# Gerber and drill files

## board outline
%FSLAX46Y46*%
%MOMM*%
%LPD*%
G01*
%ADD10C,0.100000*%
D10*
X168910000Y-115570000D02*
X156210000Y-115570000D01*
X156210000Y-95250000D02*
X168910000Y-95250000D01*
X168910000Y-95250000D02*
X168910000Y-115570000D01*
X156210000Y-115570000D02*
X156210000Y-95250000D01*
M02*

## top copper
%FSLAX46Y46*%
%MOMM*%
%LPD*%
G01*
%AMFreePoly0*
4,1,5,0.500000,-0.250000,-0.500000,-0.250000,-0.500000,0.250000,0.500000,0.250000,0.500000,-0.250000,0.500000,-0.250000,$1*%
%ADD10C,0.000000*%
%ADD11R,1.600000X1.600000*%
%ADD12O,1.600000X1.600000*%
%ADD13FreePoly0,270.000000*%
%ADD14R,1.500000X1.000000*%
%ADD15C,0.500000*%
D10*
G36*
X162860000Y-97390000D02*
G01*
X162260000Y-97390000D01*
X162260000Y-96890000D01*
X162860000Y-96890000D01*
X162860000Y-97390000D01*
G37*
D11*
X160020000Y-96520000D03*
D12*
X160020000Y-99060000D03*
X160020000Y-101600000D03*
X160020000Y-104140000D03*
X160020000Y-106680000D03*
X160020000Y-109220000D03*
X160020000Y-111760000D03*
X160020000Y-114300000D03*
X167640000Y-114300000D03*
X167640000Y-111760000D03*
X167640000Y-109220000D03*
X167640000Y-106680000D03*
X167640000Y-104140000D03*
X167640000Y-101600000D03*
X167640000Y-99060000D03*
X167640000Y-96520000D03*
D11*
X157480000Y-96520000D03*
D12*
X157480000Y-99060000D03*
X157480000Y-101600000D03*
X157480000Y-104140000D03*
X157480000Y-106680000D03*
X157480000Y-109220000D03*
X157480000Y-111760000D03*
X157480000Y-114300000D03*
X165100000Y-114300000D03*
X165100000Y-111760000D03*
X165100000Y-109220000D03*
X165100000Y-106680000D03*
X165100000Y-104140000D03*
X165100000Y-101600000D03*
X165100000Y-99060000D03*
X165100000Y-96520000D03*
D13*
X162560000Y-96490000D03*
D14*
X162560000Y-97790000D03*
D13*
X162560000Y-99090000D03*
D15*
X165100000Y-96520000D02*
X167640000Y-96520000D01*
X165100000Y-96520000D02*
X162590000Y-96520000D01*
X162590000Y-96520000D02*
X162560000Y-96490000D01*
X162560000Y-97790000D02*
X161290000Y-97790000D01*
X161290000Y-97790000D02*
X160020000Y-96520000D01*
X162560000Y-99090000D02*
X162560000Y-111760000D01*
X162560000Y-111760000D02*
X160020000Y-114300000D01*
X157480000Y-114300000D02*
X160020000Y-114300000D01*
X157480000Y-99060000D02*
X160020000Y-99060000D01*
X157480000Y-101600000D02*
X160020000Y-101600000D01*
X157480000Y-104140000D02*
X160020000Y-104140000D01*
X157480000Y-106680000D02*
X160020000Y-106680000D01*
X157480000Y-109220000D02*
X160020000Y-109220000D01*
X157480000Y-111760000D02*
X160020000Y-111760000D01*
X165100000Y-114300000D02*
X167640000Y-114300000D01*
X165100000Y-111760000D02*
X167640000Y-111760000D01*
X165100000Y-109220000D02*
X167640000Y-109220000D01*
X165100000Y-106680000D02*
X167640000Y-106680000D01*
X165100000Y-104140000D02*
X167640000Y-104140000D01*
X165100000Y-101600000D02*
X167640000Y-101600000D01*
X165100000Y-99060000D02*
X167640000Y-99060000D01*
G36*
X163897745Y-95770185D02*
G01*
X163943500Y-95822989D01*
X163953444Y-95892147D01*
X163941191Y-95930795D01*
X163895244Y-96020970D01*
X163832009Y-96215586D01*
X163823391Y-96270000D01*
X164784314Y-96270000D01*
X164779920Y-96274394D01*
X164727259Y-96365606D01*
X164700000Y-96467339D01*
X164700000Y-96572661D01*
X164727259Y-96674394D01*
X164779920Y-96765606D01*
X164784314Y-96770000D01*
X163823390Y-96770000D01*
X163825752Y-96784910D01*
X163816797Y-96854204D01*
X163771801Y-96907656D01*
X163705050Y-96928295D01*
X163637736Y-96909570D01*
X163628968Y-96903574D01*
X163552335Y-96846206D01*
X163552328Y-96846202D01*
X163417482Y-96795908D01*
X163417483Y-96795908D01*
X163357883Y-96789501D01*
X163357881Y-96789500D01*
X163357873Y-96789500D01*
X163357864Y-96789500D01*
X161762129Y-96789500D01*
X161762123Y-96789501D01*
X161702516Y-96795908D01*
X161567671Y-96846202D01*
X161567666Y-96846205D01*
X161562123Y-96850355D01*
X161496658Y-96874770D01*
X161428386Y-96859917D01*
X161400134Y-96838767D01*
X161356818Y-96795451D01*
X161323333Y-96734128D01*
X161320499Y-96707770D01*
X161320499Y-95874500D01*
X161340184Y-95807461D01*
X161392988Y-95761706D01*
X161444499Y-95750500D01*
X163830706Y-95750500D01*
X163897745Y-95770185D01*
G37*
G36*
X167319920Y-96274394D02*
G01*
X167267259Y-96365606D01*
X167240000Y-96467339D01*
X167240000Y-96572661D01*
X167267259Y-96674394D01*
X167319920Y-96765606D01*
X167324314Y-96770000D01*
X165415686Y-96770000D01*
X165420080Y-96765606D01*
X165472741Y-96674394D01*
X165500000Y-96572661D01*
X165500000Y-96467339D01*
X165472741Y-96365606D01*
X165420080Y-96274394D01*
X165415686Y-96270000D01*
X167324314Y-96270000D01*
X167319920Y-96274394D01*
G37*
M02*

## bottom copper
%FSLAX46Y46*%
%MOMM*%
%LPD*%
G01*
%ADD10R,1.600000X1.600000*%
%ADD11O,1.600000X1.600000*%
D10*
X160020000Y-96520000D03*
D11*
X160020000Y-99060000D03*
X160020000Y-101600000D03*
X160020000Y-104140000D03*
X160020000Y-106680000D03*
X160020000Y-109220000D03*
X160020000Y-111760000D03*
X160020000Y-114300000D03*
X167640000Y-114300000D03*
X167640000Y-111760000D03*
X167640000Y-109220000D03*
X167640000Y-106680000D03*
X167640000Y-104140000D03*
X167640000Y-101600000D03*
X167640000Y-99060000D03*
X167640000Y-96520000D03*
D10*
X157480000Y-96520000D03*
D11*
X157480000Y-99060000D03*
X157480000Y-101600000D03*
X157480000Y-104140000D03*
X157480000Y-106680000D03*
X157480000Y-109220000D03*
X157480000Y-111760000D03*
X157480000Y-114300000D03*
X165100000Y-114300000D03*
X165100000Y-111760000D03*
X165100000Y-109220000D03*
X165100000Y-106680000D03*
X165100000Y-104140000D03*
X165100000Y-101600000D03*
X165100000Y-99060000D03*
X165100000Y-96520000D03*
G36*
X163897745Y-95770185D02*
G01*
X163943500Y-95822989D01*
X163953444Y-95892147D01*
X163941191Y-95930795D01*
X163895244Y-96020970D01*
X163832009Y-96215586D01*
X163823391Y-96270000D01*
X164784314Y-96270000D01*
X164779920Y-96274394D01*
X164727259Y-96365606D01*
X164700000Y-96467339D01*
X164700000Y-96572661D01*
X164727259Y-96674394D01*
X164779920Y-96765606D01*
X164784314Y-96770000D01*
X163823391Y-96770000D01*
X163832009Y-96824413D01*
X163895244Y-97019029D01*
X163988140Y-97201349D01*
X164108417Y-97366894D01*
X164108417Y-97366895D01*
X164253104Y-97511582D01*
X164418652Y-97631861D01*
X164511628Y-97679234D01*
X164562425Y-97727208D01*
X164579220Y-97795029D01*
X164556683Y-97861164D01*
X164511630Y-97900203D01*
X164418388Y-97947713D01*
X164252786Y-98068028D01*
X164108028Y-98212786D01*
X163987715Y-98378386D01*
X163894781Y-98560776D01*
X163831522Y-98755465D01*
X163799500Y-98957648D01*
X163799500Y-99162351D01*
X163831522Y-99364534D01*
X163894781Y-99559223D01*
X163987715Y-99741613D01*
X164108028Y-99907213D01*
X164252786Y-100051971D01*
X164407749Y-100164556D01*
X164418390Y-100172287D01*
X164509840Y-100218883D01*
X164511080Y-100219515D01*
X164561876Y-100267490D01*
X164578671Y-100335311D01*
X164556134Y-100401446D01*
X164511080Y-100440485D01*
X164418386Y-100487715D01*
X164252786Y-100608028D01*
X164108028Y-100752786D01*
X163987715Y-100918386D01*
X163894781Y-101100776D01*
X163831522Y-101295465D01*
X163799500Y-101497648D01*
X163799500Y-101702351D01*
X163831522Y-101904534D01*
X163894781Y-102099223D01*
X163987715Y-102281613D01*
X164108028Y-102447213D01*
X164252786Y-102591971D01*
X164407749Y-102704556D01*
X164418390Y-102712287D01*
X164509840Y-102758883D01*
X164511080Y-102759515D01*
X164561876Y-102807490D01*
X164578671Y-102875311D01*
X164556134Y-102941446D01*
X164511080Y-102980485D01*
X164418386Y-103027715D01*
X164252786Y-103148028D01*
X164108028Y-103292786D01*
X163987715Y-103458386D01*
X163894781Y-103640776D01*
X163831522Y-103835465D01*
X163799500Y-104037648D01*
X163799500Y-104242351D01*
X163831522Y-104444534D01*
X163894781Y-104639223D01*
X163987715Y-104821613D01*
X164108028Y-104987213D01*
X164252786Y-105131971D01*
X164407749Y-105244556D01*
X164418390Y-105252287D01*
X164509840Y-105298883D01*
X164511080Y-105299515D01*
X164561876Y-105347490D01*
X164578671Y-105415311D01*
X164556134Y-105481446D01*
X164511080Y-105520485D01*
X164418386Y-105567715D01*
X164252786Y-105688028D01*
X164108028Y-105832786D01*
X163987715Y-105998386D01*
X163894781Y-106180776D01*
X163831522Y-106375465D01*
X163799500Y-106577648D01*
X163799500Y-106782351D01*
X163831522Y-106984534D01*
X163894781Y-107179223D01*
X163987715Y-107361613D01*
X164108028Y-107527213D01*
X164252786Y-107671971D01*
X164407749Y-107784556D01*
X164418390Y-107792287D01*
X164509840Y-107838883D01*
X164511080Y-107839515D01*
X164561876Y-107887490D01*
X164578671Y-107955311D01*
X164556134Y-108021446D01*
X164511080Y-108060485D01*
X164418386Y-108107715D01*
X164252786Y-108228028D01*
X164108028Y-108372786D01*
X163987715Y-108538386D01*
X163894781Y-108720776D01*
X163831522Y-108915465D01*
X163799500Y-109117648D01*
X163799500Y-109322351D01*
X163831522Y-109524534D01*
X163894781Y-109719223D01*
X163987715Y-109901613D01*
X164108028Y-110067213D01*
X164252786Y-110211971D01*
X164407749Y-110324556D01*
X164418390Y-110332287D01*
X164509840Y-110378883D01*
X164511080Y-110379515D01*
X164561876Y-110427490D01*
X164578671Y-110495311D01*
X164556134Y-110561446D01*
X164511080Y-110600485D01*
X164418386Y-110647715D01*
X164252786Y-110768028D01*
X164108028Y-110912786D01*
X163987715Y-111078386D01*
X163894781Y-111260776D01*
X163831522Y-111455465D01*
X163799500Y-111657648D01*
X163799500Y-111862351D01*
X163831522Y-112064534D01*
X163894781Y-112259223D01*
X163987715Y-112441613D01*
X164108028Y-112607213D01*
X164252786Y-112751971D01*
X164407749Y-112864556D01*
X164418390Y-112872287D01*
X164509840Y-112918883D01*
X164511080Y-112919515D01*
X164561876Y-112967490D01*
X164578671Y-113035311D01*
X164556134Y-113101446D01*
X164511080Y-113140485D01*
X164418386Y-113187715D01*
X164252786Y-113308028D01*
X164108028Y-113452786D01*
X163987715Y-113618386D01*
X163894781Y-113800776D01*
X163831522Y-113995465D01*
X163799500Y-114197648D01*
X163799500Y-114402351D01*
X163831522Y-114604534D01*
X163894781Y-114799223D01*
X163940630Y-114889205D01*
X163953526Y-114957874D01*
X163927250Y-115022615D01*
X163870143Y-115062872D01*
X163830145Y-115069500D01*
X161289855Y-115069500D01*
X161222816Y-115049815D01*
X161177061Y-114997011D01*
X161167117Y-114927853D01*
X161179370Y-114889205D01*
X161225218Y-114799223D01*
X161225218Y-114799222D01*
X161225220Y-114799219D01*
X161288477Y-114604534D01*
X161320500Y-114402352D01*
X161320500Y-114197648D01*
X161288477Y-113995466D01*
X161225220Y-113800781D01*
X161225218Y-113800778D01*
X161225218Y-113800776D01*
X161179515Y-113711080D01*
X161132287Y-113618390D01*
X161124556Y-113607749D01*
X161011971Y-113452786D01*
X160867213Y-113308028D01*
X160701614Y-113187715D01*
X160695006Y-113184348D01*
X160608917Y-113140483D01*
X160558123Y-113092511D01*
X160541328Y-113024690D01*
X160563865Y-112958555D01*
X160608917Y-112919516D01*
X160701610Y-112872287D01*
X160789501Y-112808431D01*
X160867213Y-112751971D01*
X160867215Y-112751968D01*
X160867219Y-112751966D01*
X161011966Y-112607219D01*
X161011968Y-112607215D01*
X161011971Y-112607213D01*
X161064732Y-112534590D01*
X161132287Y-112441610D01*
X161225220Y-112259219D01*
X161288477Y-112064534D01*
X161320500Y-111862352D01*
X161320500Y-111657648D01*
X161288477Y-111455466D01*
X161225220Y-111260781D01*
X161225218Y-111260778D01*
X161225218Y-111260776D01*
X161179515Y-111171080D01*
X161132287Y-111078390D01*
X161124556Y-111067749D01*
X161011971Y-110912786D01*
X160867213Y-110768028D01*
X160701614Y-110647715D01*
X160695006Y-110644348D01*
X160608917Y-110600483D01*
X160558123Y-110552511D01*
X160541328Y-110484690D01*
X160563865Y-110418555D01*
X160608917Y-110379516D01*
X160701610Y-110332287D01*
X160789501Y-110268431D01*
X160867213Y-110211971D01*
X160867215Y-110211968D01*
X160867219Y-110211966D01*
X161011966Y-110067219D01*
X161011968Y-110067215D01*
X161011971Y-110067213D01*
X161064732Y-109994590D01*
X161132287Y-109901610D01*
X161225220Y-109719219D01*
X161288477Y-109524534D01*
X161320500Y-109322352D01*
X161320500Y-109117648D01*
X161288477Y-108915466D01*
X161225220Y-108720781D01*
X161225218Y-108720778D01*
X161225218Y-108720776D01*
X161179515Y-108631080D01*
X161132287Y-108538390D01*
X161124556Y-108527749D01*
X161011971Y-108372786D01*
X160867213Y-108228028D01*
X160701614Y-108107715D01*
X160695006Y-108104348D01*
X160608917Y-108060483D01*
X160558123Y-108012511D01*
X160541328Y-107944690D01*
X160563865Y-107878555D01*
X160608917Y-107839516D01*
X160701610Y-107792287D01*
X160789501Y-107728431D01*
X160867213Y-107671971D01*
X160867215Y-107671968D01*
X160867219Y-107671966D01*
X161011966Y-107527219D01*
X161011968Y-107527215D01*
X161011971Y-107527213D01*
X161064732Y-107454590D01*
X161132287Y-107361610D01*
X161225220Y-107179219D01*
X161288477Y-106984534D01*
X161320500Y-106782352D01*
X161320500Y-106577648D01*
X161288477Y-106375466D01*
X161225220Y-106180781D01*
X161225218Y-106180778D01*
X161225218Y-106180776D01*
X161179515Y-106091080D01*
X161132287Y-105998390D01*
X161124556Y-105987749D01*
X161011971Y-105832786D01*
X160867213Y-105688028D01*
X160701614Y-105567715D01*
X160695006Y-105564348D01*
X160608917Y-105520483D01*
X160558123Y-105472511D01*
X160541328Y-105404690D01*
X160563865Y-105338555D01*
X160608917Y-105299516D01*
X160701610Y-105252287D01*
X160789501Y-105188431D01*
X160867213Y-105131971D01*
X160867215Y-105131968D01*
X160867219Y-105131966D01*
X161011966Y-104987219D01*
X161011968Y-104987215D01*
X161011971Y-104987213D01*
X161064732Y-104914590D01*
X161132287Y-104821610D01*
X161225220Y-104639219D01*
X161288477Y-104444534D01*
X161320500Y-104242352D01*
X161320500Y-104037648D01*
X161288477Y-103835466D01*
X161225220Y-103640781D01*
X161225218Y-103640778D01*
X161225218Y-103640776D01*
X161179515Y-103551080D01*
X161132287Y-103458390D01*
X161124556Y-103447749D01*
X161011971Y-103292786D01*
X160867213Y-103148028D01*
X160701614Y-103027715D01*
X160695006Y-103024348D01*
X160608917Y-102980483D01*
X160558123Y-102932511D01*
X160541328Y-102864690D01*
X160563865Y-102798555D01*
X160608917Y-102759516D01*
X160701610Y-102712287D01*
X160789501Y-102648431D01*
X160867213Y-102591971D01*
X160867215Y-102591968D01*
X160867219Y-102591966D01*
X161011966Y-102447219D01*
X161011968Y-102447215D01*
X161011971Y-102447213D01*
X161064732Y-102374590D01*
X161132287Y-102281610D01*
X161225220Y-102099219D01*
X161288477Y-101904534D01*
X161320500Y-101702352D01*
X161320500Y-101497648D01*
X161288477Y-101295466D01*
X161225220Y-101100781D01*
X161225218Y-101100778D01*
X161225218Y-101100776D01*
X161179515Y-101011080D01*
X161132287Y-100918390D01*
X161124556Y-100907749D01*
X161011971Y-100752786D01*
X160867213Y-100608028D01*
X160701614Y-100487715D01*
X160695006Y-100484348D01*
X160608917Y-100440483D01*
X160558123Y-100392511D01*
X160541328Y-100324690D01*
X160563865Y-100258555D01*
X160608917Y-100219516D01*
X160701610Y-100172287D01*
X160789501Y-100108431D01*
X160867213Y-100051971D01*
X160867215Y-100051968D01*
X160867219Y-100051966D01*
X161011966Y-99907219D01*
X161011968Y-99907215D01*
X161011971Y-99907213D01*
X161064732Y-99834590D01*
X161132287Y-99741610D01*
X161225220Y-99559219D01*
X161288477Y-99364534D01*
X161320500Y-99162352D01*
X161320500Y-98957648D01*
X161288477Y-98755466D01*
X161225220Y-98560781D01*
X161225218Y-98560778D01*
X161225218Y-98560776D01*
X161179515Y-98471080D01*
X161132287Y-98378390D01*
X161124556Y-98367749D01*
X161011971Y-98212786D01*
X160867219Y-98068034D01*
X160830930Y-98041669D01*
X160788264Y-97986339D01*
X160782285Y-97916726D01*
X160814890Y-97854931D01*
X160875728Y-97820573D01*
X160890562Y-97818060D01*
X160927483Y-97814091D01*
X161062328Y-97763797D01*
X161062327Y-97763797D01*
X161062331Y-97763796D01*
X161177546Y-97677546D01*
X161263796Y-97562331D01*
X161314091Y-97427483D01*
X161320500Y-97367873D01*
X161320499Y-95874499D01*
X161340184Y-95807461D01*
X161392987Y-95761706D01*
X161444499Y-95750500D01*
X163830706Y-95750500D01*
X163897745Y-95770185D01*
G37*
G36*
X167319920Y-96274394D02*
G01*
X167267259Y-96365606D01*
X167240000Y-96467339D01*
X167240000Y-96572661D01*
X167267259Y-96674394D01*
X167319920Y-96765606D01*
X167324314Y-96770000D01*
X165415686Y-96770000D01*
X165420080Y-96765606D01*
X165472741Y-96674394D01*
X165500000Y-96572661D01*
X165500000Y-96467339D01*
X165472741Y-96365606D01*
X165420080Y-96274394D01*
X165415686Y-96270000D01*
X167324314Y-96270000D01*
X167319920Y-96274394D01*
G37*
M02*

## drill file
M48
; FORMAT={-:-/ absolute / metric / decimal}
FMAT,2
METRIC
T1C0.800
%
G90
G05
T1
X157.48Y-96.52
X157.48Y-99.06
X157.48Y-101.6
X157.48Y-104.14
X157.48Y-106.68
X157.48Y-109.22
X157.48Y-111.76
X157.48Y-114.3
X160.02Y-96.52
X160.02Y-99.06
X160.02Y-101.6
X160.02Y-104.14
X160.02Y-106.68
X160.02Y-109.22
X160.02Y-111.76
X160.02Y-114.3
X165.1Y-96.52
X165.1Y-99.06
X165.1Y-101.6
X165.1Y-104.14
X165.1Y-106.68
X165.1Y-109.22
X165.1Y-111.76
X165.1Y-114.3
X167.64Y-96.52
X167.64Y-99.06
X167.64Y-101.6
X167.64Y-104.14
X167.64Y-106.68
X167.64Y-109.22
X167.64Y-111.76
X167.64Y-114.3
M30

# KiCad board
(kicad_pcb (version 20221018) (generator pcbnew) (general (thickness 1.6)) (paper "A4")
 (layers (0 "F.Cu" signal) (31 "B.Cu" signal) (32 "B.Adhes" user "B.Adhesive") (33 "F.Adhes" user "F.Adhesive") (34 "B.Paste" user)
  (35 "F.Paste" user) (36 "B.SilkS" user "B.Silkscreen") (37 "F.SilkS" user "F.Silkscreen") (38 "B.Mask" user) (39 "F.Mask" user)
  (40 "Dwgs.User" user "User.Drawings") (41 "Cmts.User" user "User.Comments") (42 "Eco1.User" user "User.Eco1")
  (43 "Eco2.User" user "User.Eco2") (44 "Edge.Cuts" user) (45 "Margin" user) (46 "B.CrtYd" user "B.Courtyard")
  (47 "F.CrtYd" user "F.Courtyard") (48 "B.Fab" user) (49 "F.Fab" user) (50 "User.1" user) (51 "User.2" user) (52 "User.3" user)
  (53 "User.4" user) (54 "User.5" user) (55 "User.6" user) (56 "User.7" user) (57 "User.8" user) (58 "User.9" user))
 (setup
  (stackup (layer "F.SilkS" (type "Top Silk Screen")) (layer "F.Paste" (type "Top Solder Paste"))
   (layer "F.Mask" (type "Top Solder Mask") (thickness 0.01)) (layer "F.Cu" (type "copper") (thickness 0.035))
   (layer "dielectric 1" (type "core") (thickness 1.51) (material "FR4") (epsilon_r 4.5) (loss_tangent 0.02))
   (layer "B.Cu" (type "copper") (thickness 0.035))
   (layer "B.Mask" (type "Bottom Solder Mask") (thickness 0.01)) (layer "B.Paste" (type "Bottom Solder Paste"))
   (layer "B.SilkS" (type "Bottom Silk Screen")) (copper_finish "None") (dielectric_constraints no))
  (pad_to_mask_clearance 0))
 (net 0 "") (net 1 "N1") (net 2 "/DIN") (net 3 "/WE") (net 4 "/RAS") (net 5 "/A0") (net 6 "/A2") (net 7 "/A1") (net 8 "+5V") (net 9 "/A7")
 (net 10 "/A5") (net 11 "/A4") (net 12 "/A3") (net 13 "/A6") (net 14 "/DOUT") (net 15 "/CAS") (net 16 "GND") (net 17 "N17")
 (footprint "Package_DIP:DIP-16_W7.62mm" (layer "F.Cu") (at 160.02 96.52)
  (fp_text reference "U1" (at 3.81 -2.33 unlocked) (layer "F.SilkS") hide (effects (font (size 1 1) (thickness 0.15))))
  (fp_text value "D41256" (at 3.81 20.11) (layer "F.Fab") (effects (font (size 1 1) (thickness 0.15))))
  (pad "1" thru_hole rect (at 0 0) (size 1.6 1.6) (drill 0.8) (layers "*.Cu" "*.Mask") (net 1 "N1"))
  (pad "2" thru_hole oval (at 0 2.54) (size 1.6 1.6) (drill 0.8) (layers "*.Cu" "*.Mask") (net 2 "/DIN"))
  (pad "3" thru_hole oval (at 0 5.08) (size 1.6 1.6) (drill 0.8) (layers "*.Cu" "*.Mask") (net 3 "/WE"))
  (pad "4" thru_hole oval (at 0 7.62) (size 1.6 1.6) (drill 0.8) (layers "*.Cu" "*.Mask") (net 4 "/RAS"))
  (pad "5" thru_hole oval (at 0 10.16) (size 1.6 1.6) (drill 0.8) (layers "*.Cu" "*.Mask") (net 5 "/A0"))
  (pad "6" thru_hole oval (at 0 12.7) (size 1.6 1.6) (drill 0.8) (layers "*.Cu" "*.Mask") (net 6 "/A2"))
  (pad "7" thru_hole oval (at 0 15.24) (size 1.6 1.6) (drill 0.8) (layers "*.Cu" "*.Mask") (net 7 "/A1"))
  (pad "8" thru_hole oval (at 0 17.78) (size 1.6 1.6) (drill 0.8) (layers "*.Cu" "*.Mask") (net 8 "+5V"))
  (pad "9" thru_hole oval (at 7.62 17.78) (size 1.6 1.6) (drill 0.8) (layers "*.Cu" "*.Mask") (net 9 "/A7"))
  (pad "10" thru_hole oval (at 7.62 15.24) (size 1.6 1.6) (drill 0.8) (layers "*.Cu" "*.Mask") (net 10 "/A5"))
  (pad "11" thru_hole oval (at 7.62 12.7) (size 1.6 1.6) (drill 0.8) (layers "*.Cu" "*.Mask") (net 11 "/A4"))
  (pad "12" thru_hole oval (at 7.62 10.16) (size 1.6 1.6) (drill 0.8) (layers "*.Cu" "*.Mask") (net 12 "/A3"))
  (pad "13" thru_hole oval (at 7.62 7.62) (size 1.6 1.6) (drill 0.8) (layers "*.Cu" "*.Mask") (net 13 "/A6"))
  (pad "14" thru_hole oval (at 7.62 5.08) (size 1.6 1.6) (drill 0.8) (layers "*.Cu" "*.Mask") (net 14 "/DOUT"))
  (pad "15" thru_hole oval (at 7.62 2.54) (size 1.6 1.6) (drill 0.8) (layers "*.Cu" "*.Mask") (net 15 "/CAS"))
  (pad "16" thru_hole oval (at 7.62 0) (size 1.6 1.6) (drill 0.8) (layers "*.Cu" "*.Mask") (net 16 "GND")))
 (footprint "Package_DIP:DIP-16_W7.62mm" (layer "F.Cu") (at 157.48 96.52)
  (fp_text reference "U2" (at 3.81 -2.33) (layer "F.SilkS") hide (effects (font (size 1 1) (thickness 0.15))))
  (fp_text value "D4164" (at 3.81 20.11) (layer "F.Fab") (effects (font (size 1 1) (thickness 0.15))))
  (pad "1" thru_hole rect (at 0 0) (size 1.6 1.6) (drill 0.8) (layers "*.Cu" "*.Mask") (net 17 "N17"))
  (pad "2" thru_hole oval (at 0 2.54) (size 1.6 1.6) (drill 0.8) (layers "*.Cu" "*.Mask") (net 2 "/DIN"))
  (pad "3" thru_hole oval (at 0 5.08) (size 1.6 1.6) (drill 0.8) (layers "*.Cu" "*.Mask") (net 3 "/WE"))
  (pad "4" thru_hole oval (at 0 7.62) (size 1.6 1.6) (drill 0.8) (layers "*.Cu" "*.Mask") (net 4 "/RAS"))
  (pad "5" thru_hole oval (at 0 10.16) (size 1.6 1.6) (drill 0.8) (layers "*.Cu" "*.Mask") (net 5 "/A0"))
  (pad "6" thru_hole oval (at 0 12.7) (size 1.6 1.6) (drill 0.8) (layers "*.Cu" "*.Mask") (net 6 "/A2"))
  (pad "7" thru_hole oval (at 0 15.24) (size 1.6 1.6) (drill 0.8) (layers "*.Cu" "*.Mask") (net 7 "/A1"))
  (pad "8" thru_hole oval (at 0 17.78) (size 1.6 1.6) (drill 0.8) (layers "*.Cu" "*.Mask") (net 8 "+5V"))
  (pad "9" thru_hole oval (at 7.62 17.78) (size 1.6 1.6) (drill 0.8) (layers "*.Cu" "*.Mask") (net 9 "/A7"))
  (pad "10" thru_hole oval (at 7.62 15.24) (size 1.6 1.6) (drill 0.8) (layers "*.Cu" "*.Mask") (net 10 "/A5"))
  (pad "11" thru_hole oval (at 7.62 12.7) (size 1.6 1.6) (drill 0.8) (layers "*.Cu" "*.Mask") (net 11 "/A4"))
  (pad "12" thru_hole oval (at 7.62 10.16) (size 1.6 1.6) (drill 0.8) (layers "*.Cu" "*.Mask") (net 12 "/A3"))
  (pad "13" thru_hole oval (at 7.62 7.62) (size 1.6 1.6) (drill 0.8) (layers "*.Cu" "*.Mask") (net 13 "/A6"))
  (pad "14" thru_hole oval (at 7.62 5.08) (size 1.6 1.6) (drill 0.8) (layers "*.Cu" "*.Mask") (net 14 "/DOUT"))
  (pad "15" thru_hole oval (at 7.62 2.54) (size 1.6 1.6) (drill 0.8) (layers "*.Cu" "*.Mask") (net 15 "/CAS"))
  (pad "16" thru_hole oval (at 7.62 0) (size 1.6 1.6) (drill 0.8) (layers "*.Cu" "*.Mask") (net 16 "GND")))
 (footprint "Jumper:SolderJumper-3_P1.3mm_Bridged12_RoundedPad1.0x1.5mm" (layer "F.Cu") (at 162.56 97.79 -90) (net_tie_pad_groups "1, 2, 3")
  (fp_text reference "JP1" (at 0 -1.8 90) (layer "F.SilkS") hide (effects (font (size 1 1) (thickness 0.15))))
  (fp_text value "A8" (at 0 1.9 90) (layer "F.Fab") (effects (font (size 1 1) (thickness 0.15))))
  (fp_poly (pts (xy -0.9 -0.3) (xy -0.4 -0.3) (xy -0.4 0.3) (xy -0.9 0.3)) (stroke (width 0) (type solid)) (fill solid) (layer "F.Cu"))
  (pad "1" smd custom (at -1.3 0 270) (size 1 0.5) (layers "F.Cu" "F.Mask") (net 16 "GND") (zone_connect 2) (thermal_bridge_angle 45)
   (options (clearance outline) (anchor rect)) (primitives))
  (pad "2" smd rect (at 0 0 270) (size 1 1.5) (layers "F.Cu" "F.Mask") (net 1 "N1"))
  (pad "3" smd custom (at 1.3 0 270) (size 1 0.5) (layers "F.Cu" "F.Mask") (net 8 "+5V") (zone_connect 2) (thermal_bridge_angle 45)
   (options (clearance outline) (anchor rect)) (primitives)))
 (gr_line (start 168.91 115.57) (end 156.21 115.57) (stroke (width 0.1) (type default)) (layer "Edge.Cuts"))
 (gr_line (start 156.21 95.25) (end 168.91 95.25) (stroke (width 0.1) (type default)) (layer "Edge.Cuts"))
 (gr_line (start 168.91 95.25) (end 168.91 115.57) (stroke (width 0.1) (type default)) (layer "Edge.Cuts"))
 (gr_line (start 156.21 115.57) (end 156.21 95.25) (stroke (width 0.1) (type default)) (layer "Edge.Cuts"))
 (segment (start 165.1 96.52) (end 167.64 96.52) (width 0.5) (layer "F.Cu") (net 16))
 (segment (start 165.1 96.52) (end 162.59 96.52) (width 0.5) (layer "F.Cu") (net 16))
 (segment (start 162.59 96.52) (end 162.56 96.49) (width 0.5) (layer "F.Cu") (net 16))
 (segment (start 162.56 97.79) (end 161.29 97.79) (width 0.5) (layer "F.Cu") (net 1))
 (segment (start 161.29 97.79) (end 160.02 96.52) (width 0.5) (layer "F.Cu") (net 1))
 (segment (start 162.56 99.09) (end 162.56 111.76) (width 0.5) (layer "F.Cu") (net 8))
 (segment (start 162.56 111.76) (end 160.02 114.3) (width 0.5) (layer "F.Cu") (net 8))
 (segment (start 157.48 114.3) (end 160.02 114.3) (width 0.5) (layer "F.Cu") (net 8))
 (segment (start 157.48 99.06) (end 160.02 99.06) (width 0.5) (layer "F.Cu") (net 2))
 (segment (start 157.48 101.6) (end 160.02 101.6) (width 0.5) (layer "F.Cu") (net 3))
 (segment (start 157.48 104.14) (end 160.02 104.14) (width 0.5) (layer "F.Cu") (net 4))
 (segment (start 157.48 106.68) (end 160.02 106.68) (width 0.5) (layer "F.Cu") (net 5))
 (segment (start 157.48 109.22) (end 160.02 109.22) (width 0.5) (layer "F.Cu") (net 6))
 (segment (start 157.48 111.76) (end 160.02 111.76) (width 0.5) (layer "F.Cu") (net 7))
 (segment (start 165.1 114.3) (end 167.64 114.3) (width 0.5) (layer "F.Cu") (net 9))
 (segment (start 165.1 111.76) (end 167.64 111.76) (width 0.5) (layer "F.Cu") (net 10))
 (segment (start 165.1 109.22) (end 167.64 109.22) (width 0.5) (layer "F.Cu") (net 11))
 (segment (start 165.1 106.68) (end 167.64 106.68) (width 0.5) (layer "F.Cu") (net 12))
 (segment (start 165.1 104.14) (end 167.64 104.14) (width 0.5) (layer "F.Cu") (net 13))
 (segment (start 165.1 101.6) (end 167.64 101.6) (width 0.5) (layer "F.Cu") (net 14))
 (segment (start 165.1 99.06) (end 167.64 99.06) (width 0.5) (layer "F.Cu") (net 15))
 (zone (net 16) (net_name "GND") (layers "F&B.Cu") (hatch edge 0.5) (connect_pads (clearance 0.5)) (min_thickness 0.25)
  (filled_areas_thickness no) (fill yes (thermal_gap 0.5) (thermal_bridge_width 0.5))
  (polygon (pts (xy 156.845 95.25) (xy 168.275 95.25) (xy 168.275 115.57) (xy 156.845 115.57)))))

